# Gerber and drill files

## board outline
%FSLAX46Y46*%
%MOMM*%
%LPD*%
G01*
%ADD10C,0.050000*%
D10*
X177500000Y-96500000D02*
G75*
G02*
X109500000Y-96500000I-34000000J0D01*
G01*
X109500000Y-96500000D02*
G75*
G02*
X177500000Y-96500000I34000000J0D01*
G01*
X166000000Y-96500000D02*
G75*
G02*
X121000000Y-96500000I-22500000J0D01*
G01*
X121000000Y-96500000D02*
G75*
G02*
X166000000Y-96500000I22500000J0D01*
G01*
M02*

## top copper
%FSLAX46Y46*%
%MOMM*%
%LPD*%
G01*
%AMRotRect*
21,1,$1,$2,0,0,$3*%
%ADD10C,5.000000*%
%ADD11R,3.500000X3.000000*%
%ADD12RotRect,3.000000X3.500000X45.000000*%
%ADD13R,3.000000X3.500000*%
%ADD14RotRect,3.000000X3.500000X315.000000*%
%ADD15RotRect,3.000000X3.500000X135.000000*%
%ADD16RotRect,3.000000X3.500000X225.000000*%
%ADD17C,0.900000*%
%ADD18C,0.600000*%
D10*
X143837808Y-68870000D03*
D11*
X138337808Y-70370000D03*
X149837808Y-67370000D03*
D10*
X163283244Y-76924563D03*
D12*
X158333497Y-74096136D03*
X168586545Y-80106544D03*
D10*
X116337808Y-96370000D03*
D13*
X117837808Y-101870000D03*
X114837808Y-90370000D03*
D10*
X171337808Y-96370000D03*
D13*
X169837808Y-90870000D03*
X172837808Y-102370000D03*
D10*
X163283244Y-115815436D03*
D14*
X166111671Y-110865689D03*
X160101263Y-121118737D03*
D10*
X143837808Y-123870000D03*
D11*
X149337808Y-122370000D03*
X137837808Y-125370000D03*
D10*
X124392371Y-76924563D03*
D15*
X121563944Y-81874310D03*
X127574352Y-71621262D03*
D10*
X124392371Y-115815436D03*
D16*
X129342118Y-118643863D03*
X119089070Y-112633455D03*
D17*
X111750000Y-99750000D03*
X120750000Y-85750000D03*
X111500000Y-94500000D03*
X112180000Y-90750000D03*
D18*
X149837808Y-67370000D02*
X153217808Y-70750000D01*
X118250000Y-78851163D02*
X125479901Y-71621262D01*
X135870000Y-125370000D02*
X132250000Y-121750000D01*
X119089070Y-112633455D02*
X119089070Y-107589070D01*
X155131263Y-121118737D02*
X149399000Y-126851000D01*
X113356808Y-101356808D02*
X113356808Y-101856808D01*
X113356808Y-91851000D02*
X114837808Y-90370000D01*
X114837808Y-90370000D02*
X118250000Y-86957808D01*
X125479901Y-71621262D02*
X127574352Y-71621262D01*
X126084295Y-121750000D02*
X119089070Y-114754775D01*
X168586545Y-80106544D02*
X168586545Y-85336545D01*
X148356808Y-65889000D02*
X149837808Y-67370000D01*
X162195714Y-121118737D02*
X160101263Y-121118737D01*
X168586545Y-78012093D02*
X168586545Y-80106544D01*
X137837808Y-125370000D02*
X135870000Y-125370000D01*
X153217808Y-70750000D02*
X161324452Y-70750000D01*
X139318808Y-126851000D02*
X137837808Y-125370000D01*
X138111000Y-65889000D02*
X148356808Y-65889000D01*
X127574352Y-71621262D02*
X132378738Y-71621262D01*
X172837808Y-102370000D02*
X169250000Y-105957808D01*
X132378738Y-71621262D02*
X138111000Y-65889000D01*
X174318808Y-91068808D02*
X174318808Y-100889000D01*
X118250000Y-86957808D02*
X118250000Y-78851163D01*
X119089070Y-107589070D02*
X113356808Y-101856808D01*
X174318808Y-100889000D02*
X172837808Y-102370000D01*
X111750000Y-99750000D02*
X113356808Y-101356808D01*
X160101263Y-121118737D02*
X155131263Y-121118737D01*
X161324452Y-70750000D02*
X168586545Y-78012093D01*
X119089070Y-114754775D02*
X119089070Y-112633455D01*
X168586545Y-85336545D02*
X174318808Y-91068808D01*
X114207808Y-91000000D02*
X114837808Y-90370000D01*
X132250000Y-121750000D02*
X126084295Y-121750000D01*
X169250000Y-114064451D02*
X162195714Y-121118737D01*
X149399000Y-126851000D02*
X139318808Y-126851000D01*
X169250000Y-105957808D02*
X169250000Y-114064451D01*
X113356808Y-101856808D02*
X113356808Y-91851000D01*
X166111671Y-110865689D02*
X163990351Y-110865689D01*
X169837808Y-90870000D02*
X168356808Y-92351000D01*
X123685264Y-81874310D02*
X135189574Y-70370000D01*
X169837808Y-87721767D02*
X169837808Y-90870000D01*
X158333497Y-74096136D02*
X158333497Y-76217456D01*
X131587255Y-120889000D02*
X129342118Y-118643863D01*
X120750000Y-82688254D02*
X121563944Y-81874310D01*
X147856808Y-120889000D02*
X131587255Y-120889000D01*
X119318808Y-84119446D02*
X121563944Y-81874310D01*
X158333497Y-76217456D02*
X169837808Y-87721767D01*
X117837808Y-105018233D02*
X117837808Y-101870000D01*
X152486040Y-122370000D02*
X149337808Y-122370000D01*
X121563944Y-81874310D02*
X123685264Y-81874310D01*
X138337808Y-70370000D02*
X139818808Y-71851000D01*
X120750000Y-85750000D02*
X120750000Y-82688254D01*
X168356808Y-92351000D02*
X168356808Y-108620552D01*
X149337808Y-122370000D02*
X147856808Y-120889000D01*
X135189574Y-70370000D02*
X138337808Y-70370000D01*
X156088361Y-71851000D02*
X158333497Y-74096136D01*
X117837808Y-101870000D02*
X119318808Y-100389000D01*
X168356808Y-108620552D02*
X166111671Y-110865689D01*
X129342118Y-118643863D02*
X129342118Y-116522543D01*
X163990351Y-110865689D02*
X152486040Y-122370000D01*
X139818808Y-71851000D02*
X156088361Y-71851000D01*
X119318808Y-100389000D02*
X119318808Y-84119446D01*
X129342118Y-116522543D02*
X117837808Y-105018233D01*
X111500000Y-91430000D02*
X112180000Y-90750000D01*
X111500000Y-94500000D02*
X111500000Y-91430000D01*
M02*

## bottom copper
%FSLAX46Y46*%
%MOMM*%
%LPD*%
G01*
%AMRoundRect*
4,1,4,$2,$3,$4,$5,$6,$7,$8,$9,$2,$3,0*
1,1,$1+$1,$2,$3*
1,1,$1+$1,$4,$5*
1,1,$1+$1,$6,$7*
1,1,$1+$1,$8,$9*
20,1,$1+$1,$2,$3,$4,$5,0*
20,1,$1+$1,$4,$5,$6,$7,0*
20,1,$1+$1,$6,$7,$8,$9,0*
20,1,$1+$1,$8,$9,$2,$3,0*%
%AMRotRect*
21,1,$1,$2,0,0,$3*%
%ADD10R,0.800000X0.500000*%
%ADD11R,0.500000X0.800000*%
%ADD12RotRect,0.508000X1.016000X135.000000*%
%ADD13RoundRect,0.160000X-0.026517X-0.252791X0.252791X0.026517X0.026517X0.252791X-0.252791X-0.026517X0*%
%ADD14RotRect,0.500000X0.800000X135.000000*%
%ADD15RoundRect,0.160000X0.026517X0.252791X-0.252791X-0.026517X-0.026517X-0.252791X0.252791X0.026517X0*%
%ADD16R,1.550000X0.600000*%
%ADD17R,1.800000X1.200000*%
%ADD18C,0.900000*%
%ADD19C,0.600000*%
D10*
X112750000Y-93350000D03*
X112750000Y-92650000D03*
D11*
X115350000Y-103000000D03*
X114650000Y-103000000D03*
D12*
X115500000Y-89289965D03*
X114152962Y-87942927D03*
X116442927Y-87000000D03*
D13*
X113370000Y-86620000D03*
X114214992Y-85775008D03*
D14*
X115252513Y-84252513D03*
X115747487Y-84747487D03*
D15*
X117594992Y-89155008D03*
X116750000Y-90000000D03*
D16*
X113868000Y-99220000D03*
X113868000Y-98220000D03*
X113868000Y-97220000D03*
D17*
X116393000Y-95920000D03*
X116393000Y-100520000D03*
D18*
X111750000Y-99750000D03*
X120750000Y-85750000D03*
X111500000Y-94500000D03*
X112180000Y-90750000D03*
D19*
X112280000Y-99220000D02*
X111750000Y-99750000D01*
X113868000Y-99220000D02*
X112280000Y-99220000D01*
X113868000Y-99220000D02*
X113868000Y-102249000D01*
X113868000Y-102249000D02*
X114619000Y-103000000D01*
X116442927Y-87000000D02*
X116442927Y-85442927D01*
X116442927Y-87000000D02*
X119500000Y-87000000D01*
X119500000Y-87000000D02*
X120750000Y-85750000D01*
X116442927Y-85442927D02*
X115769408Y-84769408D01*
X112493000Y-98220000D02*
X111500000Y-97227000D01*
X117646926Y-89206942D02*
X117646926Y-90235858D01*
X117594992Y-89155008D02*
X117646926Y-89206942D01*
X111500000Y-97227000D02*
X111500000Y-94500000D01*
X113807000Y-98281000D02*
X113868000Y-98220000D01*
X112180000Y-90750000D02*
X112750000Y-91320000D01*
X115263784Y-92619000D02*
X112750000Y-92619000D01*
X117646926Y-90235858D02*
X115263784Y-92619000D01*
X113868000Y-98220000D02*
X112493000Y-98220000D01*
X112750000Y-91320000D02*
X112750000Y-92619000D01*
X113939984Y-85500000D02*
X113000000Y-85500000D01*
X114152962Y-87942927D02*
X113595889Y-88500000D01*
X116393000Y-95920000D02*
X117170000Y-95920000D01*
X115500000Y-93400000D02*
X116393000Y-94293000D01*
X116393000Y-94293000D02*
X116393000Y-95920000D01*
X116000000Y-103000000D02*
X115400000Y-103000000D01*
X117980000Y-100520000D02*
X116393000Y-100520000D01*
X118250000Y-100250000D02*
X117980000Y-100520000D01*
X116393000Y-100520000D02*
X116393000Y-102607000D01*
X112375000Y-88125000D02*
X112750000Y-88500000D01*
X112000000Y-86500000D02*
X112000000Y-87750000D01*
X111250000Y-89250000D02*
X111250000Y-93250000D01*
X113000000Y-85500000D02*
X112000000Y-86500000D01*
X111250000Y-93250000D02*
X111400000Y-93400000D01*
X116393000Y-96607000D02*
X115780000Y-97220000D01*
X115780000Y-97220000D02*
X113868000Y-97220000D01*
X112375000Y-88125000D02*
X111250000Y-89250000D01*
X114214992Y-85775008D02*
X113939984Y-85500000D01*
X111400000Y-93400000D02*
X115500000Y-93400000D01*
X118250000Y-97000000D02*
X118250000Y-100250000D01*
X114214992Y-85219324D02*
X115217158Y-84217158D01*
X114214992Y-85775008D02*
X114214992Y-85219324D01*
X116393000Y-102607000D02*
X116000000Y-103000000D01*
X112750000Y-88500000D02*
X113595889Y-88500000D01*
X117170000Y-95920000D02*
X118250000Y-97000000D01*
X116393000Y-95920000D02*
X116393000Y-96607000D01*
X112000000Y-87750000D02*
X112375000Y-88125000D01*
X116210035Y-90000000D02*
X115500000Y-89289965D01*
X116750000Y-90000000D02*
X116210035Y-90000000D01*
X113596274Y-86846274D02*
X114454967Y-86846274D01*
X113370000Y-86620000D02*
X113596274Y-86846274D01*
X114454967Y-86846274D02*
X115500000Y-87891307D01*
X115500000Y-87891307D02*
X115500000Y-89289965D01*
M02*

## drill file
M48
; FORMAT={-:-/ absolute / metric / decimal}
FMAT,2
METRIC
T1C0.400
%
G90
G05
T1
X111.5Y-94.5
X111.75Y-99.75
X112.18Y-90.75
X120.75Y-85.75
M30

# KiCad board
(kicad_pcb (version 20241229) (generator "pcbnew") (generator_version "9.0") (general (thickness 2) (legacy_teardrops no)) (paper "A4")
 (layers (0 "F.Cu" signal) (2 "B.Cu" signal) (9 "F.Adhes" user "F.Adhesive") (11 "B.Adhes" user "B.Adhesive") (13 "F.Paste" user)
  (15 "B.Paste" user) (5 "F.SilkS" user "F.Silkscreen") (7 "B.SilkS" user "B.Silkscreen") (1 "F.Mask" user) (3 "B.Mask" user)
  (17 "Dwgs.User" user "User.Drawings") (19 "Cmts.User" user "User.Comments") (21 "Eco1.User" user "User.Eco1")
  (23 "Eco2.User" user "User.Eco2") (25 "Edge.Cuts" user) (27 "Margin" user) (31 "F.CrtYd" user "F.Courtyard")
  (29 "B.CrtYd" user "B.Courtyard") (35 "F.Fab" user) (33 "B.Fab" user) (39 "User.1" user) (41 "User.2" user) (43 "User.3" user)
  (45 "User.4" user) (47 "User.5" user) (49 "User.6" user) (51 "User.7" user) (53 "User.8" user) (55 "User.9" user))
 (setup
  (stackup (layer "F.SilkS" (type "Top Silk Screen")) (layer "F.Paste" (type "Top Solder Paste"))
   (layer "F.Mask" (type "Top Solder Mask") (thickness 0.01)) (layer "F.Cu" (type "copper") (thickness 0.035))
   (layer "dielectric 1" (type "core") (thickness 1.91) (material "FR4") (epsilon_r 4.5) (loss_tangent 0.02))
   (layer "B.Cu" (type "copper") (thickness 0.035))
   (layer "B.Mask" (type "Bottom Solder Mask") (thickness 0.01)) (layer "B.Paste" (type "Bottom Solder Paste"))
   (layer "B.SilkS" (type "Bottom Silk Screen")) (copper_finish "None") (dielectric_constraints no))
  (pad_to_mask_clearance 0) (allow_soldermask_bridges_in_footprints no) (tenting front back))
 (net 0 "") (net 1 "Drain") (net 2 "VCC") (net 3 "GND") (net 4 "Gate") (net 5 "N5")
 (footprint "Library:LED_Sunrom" (layer "F.Cu") (at 143.837808 68.87)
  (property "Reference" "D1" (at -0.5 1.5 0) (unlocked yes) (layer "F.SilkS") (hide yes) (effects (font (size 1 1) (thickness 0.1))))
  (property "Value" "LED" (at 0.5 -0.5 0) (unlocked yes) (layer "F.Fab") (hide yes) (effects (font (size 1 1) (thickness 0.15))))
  (pad "" smd circle (at 0 0 90) (size 5 5) (layers "F.Cu" "F.Mask" "F.Paste") (solder_mask_margin 0.102))
  (pad "1" smd rect (at -5.5 1.5 90) (size 3 3.5) (layers "F.Cu" "F.Mask" "F.Paste") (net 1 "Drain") (solder_mask_margin 0.102))
  (pad "2" smd rect (at 6 -1.5 90) (size 3 3.5) (layers "F.Cu" "F.Mask" "F.Paste") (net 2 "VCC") (solder_mask_margin 0.102)))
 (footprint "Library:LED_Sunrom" (layer "F.Cu") (at 163.283244 76.924563 -45)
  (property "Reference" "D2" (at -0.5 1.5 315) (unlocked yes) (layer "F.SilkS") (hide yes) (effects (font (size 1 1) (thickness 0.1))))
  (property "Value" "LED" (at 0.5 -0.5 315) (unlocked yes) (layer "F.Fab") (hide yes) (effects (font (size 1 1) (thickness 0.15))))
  (pad "" smd circle (at 0 0 45) (size 5 5) (layers "F.Cu" "F.Mask" "F.Paste") (solder_mask_margin 0.102))
  (pad "1" smd rect (at -5.5 1.5 45) (size 3 3.5) (layers "F.Cu" "F.Mask" "F.Paste") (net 1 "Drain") (solder_mask_margin 0.102))
  (pad "2" smd rect (at 6 -1.5 45) (size 3 3.5) (layers "F.Cu" "F.Mask" "F.Paste") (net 2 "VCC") (solder_mask_margin 0.102)))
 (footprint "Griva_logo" (layer "F.Cu") (at 116.847808 106.51)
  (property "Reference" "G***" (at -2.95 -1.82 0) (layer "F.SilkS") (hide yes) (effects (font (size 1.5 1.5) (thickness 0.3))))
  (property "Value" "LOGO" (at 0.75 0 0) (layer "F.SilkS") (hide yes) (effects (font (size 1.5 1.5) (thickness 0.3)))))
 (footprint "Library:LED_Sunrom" (layer "F.Cu") (at 116.337808 96.37 90)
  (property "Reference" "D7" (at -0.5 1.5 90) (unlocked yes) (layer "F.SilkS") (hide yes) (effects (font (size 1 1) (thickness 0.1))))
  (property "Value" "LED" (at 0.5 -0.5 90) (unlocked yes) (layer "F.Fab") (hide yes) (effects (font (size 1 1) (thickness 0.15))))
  (pad "" smd circle (at 0 0 180) (size 5 5) (layers "F.Cu" "F.Mask" "F.Paste") (solder_mask_margin 0.102))
  (pad "1" smd rect (at -5.5 1.5 180) (size 3 3.5) (layers "F.Cu" "F.Mask" "F.Paste") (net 1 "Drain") (solder_mask_margin 0.102))
  (pad "2" smd rect (at 6 -1.5 180) (size 3 3.5) (layers "F.Cu" "F.Mask" "F.Paste") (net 2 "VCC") (solder_mask_margin 0.102)))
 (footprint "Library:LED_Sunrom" (layer "F.Cu") (at 171.337808 96.37 -90)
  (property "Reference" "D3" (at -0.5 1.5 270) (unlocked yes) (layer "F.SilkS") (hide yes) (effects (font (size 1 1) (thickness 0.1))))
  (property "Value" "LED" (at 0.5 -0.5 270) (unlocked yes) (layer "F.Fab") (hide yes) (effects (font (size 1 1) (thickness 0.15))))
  (pad "" smd circle (at 0 0) (size 5 5) (layers "F.Cu" "F.Mask" "F.Paste") (solder_mask_margin 0.102))
  (pad "1" smd rect (at -5.5 1.5) (size 3 3.5) (layers "F.Cu" "F.Mask" "F.Paste") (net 1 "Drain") (solder_mask_margin 0.102))
  (pad "2" smd rect (at 6 -1.5) (size 3 3.5) (layers "F.Cu" "F.Mask" "F.Paste") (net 2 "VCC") (solder_mask_margin 0.102)))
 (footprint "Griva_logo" (layer "F.Cu") (at 23.59 18.28)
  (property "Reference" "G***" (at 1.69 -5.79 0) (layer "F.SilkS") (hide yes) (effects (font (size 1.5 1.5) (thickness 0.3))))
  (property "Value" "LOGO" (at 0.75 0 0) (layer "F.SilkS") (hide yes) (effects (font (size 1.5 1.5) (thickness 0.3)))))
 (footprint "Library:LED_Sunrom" (layer "F.Cu") (at 163.283244 115.815436 -135)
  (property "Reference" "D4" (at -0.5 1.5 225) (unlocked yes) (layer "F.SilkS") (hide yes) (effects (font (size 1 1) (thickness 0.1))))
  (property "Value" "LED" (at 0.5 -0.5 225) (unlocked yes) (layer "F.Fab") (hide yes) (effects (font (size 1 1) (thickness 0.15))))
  (pad "" smd circle (at 0 0 315) (size 5 5) (layers "F.Cu" "F.Mask" "F.Paste") (solder_mask_margin 0.102))
  (pad "1" smd rect (at -5.5 1.5 315) (size 3 3.5) (layers "F.Cu" "F.Mask" "F.Paste") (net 1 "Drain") (solder_mask_margin 0.102))
  (pad "2" smd rect (at 6 -1.5 315) (size 3 3.5) (layers "F.Cu" "F.Mask" "F.Paste") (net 2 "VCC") (solder_mask_margin 0.102)))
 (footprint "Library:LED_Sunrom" (layer "F.Cu") (at 143.837808 123.87 180)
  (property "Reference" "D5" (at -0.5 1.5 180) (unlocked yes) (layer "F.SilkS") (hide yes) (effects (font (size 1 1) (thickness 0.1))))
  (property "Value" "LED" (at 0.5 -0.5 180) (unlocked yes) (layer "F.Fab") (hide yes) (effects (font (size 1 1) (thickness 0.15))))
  (pad "" smd circle (at 0 0 270) (size 5 5) (layers "F.Cu" "F.Mask" "F.Paste") (solder_mask_margin 0.102))
  (pad "1" smd rect (at -5.5 1.5 270) (size 3 3.5) (layers "F.Cu" "F.Mask" "F.Paste") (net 1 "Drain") (solder_mask_margin 0.102))
  (pad "2" smd rect (at 6 -1.5 270) (size 3 3.5) (layers "F.Cu" "F.Mask" "F.Paste") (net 2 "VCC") (solder_mask_margin 0.102)))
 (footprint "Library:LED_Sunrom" (layer "F.Cu") (at 124.392371 76.924563 45)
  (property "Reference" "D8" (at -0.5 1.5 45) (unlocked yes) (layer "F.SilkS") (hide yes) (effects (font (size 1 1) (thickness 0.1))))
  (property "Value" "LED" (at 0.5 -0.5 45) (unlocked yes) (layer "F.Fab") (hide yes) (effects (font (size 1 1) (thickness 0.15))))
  (pad "" smd circle (at 0 0 135) (size 5 5) (layers "F.Cu" "F.Mask" "F.Paste") (solder_mask_margin 0.102))
  (pad "1" smd rect (at -5.5 1.5 135) (size 3 3.5) (layers "F.Cu" "F.Mask" "F.Paste") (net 1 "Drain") (solder_mask_margin 0.102))
  (pad "2" smd rect (at 6 -1.5 135) (size 3 3.5) (layers "F.Cu" "F.Mask" "F.Paste") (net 2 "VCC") (solder_mask_margin 0.102)))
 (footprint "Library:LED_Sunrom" (layer "F.Cu") (at 124.392371 115.815436 135)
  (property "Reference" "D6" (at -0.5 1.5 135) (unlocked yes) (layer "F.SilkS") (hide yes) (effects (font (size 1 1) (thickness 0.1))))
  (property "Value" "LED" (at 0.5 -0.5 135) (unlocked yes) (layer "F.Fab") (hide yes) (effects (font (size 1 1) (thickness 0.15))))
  (pad "" smd circle (at 0 0 225) (size 5 5) (layers "F.Cu" "F.Mask" "F.Paste") (solder_mask_margin 0.102))
  (pad "1" smd rect (at -5.5 1.5 225) (size 3 3.5) (layers "F.Cu" "F.Mask" "F.Paste") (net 1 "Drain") (solder_mask_margin 0.102))
  (pad "2" smd rect (at 6 -1.5 225) (size 3 3.5) (layers "F.Cu" "F.Mask" "F.Paste") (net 2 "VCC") (solder_mask_margin 0.102)))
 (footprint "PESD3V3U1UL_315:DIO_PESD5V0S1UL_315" (layer "B.Cu") (at 112.75 93 -90)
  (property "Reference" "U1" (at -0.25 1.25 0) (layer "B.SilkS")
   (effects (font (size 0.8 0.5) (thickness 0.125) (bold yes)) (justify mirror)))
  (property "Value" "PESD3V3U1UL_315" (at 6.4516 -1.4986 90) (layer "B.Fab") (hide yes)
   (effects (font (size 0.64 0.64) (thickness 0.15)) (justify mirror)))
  (pad "A" smd rect (at 0.35 0 270) (size 0.5 0.8) (layers "B.Cu") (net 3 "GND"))
  (pad "K" smd rect (at -0.35 0 270) (size 0.5 0.8) (layers "B.Cu") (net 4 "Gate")))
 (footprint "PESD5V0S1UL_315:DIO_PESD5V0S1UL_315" (layer "B.Cu") (at 115 103)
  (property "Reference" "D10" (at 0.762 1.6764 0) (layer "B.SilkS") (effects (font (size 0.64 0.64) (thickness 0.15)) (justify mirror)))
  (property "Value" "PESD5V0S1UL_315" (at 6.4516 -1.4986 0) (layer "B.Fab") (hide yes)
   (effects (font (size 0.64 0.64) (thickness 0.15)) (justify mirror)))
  (pad "A" smd rect (at 0.35 0) (size 0.5 0.8) (layers "B.Cu") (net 3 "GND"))
  (pad "K" smd rect (at -0.35 0) (size 0.5 0.8) (layers "B.Cu") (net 2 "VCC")))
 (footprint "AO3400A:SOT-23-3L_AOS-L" (layer "B.Cu") (at 115.634704 87.808223 135)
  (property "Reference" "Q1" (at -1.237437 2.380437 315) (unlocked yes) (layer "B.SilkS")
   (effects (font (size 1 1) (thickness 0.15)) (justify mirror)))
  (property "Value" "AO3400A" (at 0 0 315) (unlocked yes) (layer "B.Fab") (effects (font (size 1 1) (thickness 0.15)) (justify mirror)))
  (pad "1" smd rect (at -0.9525 -1.143 135) (size 0.508 1.016) (layers "B.Cu" "B.Mask" "B.Paste") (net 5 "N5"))
  (pad "2" smd rect (at 0.9525 -1.143 135) (size 0.508 1.016) (layers "B.Cu" "B.Mask" "B.Paste") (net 3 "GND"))
  (pad "3" smd rect (at 0 1.143 135) (size 0.508 1.016) (layers "B.Cu" "B.Mask" "B.Paste") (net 1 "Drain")))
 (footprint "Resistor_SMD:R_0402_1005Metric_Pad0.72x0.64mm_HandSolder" (layer "B.Cu") (at 113.792496 86.197504 45)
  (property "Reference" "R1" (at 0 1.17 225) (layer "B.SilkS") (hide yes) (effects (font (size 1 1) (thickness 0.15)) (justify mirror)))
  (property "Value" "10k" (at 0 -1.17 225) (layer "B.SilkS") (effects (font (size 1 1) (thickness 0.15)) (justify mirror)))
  (pad "1" smd roundrect (at -0.5975 0 45) (size 0.715 0.64) (layers "B.Cu" "B.Mask" "B.Paste") (roundrect_rratio 0.25) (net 5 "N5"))
  (pad "2" smd roundrect (at 0.5975 0 45) (size 0.715 0.64) (layers "B.Cu" "B.Mask" "B.Paste") (roundrect_rratio 0.25) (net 3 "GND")))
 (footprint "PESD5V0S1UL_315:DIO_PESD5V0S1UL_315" (layer "B.Cu") (at 115.5 84.5 135)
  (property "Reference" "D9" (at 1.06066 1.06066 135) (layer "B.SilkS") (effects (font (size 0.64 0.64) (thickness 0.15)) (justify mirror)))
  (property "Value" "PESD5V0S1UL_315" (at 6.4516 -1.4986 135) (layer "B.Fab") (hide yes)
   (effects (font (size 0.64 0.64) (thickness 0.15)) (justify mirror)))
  (pad "A" smd rect (at 0.349999 0 135) (size 0.5 0.8) (layers "B.Cu") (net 3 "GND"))
  (pad "K" smd rect (at -0.349999 0 135) (size 0.5 0.8) (layers "B.Cu") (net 1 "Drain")))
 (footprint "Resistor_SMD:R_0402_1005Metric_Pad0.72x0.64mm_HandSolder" (layer "B.Cu") (at 117.172496 89.577504 -135)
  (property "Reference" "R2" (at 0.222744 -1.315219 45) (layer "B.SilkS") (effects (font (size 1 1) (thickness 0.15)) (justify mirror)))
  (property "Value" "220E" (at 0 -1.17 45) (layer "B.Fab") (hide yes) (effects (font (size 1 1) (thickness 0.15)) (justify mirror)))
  (pad "1" smd roundrect (at -0.5975 0 225) (size 0.715 0.64) (layers "B.Cu" "B.Mask" "B.Paste") (roundrect_rratio 0.25) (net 4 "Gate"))
  (pad "2" smd roundrect (at 0.5975 0 225) (size 0.715 0.64) (layers "B.Cu" "B.Mask" "B.Paste") (roundrect_rratio 0.25) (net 5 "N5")))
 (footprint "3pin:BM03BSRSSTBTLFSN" (layer "B.Cu") (at 115.48 98.22 -90)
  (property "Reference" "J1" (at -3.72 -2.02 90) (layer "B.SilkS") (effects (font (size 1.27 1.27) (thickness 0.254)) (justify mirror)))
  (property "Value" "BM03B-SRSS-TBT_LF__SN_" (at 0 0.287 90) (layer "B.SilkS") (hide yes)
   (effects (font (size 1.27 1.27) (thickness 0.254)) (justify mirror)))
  (pad "1" smd rect (at 1 1.612 270) (size 0.6 1.55) (layers "B.Cu" "B.Mask" "B.Paste") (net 2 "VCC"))
  (pad "2" smd rect (at 0 1.612 270) (size 0.6 1.55) (layers "B.Cu" "B.Mask" "B.Paste") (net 4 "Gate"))
  (pad "3" smd rect (at -1 1.612 270) (size 0.6 1.55) (layers "B.Cu" "B.Mask" "B.Paste") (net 3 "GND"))
  (pad "4" smd rect (at -2.3 -0.913 270) (size 1.2 1.8) (layers "B.Cu" "B.Mask" "B.Paste") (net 3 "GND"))
  (pad "5" smd rect (at 2.3 -0.913 270) (size 1.2 1.8) (layers "B.Cu" "B.Mask" "B.Paste") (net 3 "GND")))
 (gr_circle (center 143.5 96.5) (end 177.5 96.5) (stroke (width 0.05) (type solid)) (fill no) (layer "Edge.Cuts"))
 (gr_circle (center 143.5 96.5) (end 166 96.5) (stroke (width 0.05) (type default)) (fill no) (layer "Edge.Cuts"))
 (segment (start 149.837808 67.37) (end 153.217808 70.75) (width 0.6) (layer "F.Cu") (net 2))
 (segment (start 118.25 78.851163) (end 125.479901 71.621262) (width 0.6) (layer "F.Cu") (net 2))
 (segment (start 135.87 125.37) (end 132.25 121.75) (width 0.6) (layer "F.Cu") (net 2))
 (segment (start 119.08907 112.633455) (end 119.08907 107.58907) (width 0.6) (layer "F.Cu") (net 2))
 (segment (start 155.131263 121.118737) (end 149.399 126.851) (width 0.6) (layer "F.Cu") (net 2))
 (segment (start 113.356808 101.356808) (end 113.356808 101.856808) (width 0.6) (layer "F.Cu") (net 2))
 (segment (start 113.356808 91.851) (end 114.837808 90.37) (width 0.6) (layer "F.Cu") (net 2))
 (segment (start 114.837808 90.37) (end 118.25 86.957808) (width 0.6) (layer "F.Cu") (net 2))
 (segment (start 125.479901 71.621262) (end 127.574352 71.621262) (width 0.6) (layer "F.Cu") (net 2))
 (segment (start 126.084295 121.75) (end 119.08907 114.754775) (width 0.6) (layer "F.Cu") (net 2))
 (segment (start 168.586545 80.106544) (end 168.586545 85.336545) (width 0.6) (layer "F.Cu") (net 2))
 (segment (start 148.356808 65.889) (end 149.837808 67.37) (width 0.6) (layer "F.Cu") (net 2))
 (segment (start 162.195714 121.118737) (end 160.101263 121.118737) (width 0.6) (layer "F.Cu") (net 2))
 (segment (start 168.586545 78.012093) (end 168.586545 80.106544) (width 0.6) (layer "F.Cu") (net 2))
 (segment (start 137.837808 125.37) (end 135.87 125.37) (width 0.6) (layer "F.Cu") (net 2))
 (segment (start 153.217808 70.75) (end 161.324452 70.75) (width 0.6) (layer "F.Cu") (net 2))
 (segment (start 139.318808 126.851) (end 137.837808 125.37) (width 0.6) (layer "F.Cu") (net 2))
 (segment (start 138.111 65.889) (end 148.356808 65.889) (width 0.6) (layer "F.Cu") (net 2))
 (segment (start 127.574352 71.621262) (end 132.378738 71.621262) (width 0.6) (layer "F.Cu") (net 2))
 (segment (start 172.837808 102.37) (end 169.25 105.957808) (width 0.6) (layer "F.Cu") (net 2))
 (segment (start 132.378738 71.621262) (end 138.111 65.889) (width 0.6) (layer "F.Cu") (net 2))
 (segment (start 174.318808 91.068808) (end 174.318808 100.889) (width 0.6) (layer "F.Cu") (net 2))
 (segment (start 118.25 86.957808) (end 118.25 78.851163) (width 0.6) (layer "F.Cu") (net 2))
 (segment (start 119.08907 107.58907) (end 113.356808 101.856808) (width 0.6) (layer "F.Cu") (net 2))
 (segment (start 174.318808 100.889) (end 172.837808 102.37) (width 0.6) (layer "F.Cu") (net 2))
 (segment (start 111.75 99.75) (end 113.356808 101.356808) (width 0.6) (layer "F.Cu") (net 2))
 (segment (start 160.101263 121.118737) (end 155.131263 121.118737) (width 0.6) (layer "F.Cu") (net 2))
 (segment (start 161.324452 70.75) (end 168.586545 78.012093) (width 0.6) (layer "F.Cu") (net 2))
 (segment (start 119.08907 114.754775) (end 119.08907 112.633455) (width 0.6) (layer "F.Cu") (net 2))
 (segment (start 168.586545 85.336545) (end 174.318808 91.068808) (width 0.6) (layer "F.Cu") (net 2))
 (segment (start 114.207808 91) (end 114.837808 90.37) (width 0.6) (layer "F.Cu") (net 2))
 (segment (start 132.25 121.75) (end 126.084295 121.75) (width 0.6) (layer "F.Cu") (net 2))
 (segment (start 169.25 114.064451) (end 162.195714 121.118737) (width 0.6) (layer "F.Cu") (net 2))
 (segment (start 149.399 126.851) (end 139.318808 126.851) (width 0.6) (layer "F.Cu") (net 2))
 (segment (start 169.25 105.957808) (end 169.25 114.064451) (width 0.6) (layer "F.Cu") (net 2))
 (segment (start 113.356808 101.856808) (end 113.356808 91.851) (width 0.6) (layer "F.Cu") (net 2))
 (via (at 111.75 99.75) (size 0.9) (drill 0.4) (layers "F.Cu" "B.Cu") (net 2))
 (segment (start 112.28 99.22) (end 111.75 99.75) (width 0.6) (layer "B.Cu") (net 2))
 (segment (start 113.868 99.22) (end 112.28 99.22) (width 0.6) (layer "B.Cu") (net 2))
 (segment (start 113.868 99.22) (end 113.868 102.249) (width 0.6) (layer "B.Cu") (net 2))
 (segment (start 113.868 102.249) (end 114.619 103) (width 0.6) (layer "B.Cu") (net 2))
 (segment (start 166.111671 110.865689) (end 163.990351 110.865689) (width 0.6) (layer "F.Cu") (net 1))
 (segment (start 169.837808 90.87) (end 168.356808 92.351) (width 0.6) (layer "F.Cu") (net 1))
 (segment (start 123.685264 81.87431) (end 135.189574 70.37) (width 0.6) (layer "F.Cu") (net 1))
 (segment (start 169.837808 87.721767) (end 169.837808 90.87) (width 0.6) (layer "F.Cu") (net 1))
 (segment (start 158.333497 74.096136) (end 158.333497 76.217456) (width 0.6) (layer "F.Cu") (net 1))
 (segment (start 131.587255 120.889) (end 129.342118 118.643863) (width 0.6) (layer "F.Cu") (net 1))
 (segment (start 120.75 82.688254) (end 121.563944 81.87431) (width 0.6) (layer "F.Cu") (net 1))
 (segment (start 147.856808 120.889) (end 131.587255 120.889) (width 0.6) (layer "F.Cu") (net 1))
 (segment (start 119.318808 84.119446) (end 121.563944 81.87431) (width 0.6) (layer "F.Cu") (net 1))
 (segment (start 158.333497 76.217456) (end 169.837808 87.721767) (width 0.6) (layer "F.Cu") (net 1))
 (segment (start 117.837808 105.018233) (end 117.837808 101.87) (width 0.6) (layer "F.Cu") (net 1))
 (segment (start 152.48604 122.37) (end 149.337808 122.37) (width 0.6) (layer "F.Cu") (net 1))
 (segment (start 121.563944 81.87431) (end 123.685264 81.87431) (width 0.6) (layer "F.Cu") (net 1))
 (segment (start 138.337808 70.37) (end 139.818808 71.851) (width 0.6) (layer "F.Cu") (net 1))
 (segment (start 120.75 85.75) (end 120.75 82.688254) (width 0.6) (layer "F.Cu") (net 1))
 (segment (start 168.356808 92.351) (end 168.356808 108.620552) (width 0.6) (layer "F.Cu") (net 1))
 (segment (start 149.337808 122.37) (end 147.856808 120.889) (width 0.6) (layer "F.Cu") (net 1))
 (segment (start 135.189574 70.37) (end 138.337808 70.37) (width 0.6) (layer "F.Cu") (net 1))
 (segment (start 156.088361 71.851) (end 158.333497 74.096136) (width 0.6) (layer "F.Cu") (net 1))
 (segment (start 117.837808 101.87) (end 119.318808 100.389) (width 0.6) (layer "F.Cu") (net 1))
 (segment (start 168.356808 108.620552) (end 166.111671 110.865689) (width 0.6) (layer "F.Cu") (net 1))
 (segment (start 129.342118 118.643863) (end 129.342118 116.522543) (width 0.6) (layer "F.Cu") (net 1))
 (segment (start 163.990351 110.865689) (end 152.48604 122.37) (width 0.6) (layer "F.Cu") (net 1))
 (segment (start 139.818808 71.851) (end 156.088361 71.851) (width 0.6) (layer "F.Cu") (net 1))
 (segment (start 119.318808 100.389) (end 119.318808 84.119446) (width 0.6) (layer "F.Cu") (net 1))
 (segment (start 129.342118 116.522543) (end 117.837808 105.018233) (width 0.6) (layer "F.Cu") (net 1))
 (via (at 120.75 85.75) (size 0.9) (drill 0.4) (layers "F.Cu" "B.Cu") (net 1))
 (segment (start 116.442927 87) (end 116.442927 85.442927) (width 0.6) (layer "B.Cu") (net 1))
 (segment (start 116.442927 87) (end 119.5 87) (width 0.6) (layer "B.Cu") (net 1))
 (segment (start 119.5 87) (end 120.75 85.75) (width 0.6) (layer "B.Cu") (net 1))
 (segment (start 116.442927 85.442927) (end 115.769408 84.769408) (width 0.6) (layer "B.Cu") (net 1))
 (segment (start 111.5 91.43) (end 112.18 90.75) (width 0.6) (layer "F.Cu") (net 4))
 (segment (start 111.5 94.5) (end 111.5 91.43) (width 0.6) (layer "F.Cu") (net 4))
 (via (at 111.5 94.5) (size 0.9) (drill 0.4) (layers "F.Cu" "B.Cu") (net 4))
 (via (at 112.18 90.75) (size 0.9) (drill 0.4) (layers "F.Cu" "B.Cu") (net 4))
 (segment (start 112.493 98.22) (end 111.5 97.227) (width 0.6) (layer "B.Cu") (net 4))
 (segment (start 117.646926 89.206942) (end 117.646926 90.235858) (width 0.6) (layer "B.Cu") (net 4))
 (segment (start 117.594992 89.155008) (end 117.646926 89.206942) (width 0.6) (layer "B.Cu") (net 4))
 (segment (start 111.5 97.227) (end 111.5 94.5) (width 0.6) (layer "B.Cu") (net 4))
 (segment (start 113.807 98.281) (end 113.868 98.22) (width 0.6) (layer "B.Cu") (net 4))
 (segment (start 112.18 90.75) (end 112.75 91.32) (width 0.6) (layer "B.Cu") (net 4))
 (segment (start 115.263784 92.619) (end 112.75 92.619) (width 0.6) (layer "B.Cu") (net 4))
 (segment (start 117.646926 90.235858) (end 115.263784 92.619) (width 0.6) (layer "B.Cu") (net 4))
 (segment (start 113.868 98.22) (end 112.493 98.22) (width 0.6) (layer "B.Cu") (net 4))
 (segment (start 112.75 91.32) (end 112.75 92.619) (width 0.6) (layer "B.Cu") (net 4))
 (segment (start 113.939984 85.5) (end 113 85.5) (width 0.6) (layer "B.Cu") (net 3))
 (segment (start 114.152962 87.942927) (end 113.595889 88.5) (width 0.6) (layer "B.Cu") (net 3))
 (segment (start 116.393 95.92) (end 117.17 95.92) (width 0.6) (layer "B.Cu") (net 3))
 (segment (start 115.5 93.4) (end 116.393 94.293) (width 0.6) (layer "B.Cu") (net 3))
 (segment (start 116.393 94.293) (end 116.393 95.92) (width 0.6) (layer "B.Cu") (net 3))
 (segment (start 116 103) (end 115.4 103) (width 0.6) (layer "B.Cu") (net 3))
 (segment (start 117.98 100.52) (end 116.393 100.52) (width 0.6) (layer "B.Cu") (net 3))
 (segment (start 118.25 100.25) (end 117.98 100.52) (width 0.6) (layer "B.Cu") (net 3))
 (segment (start 116.393 100.52) (end 116.393 102.607) (width 0.6) (layer "B.Cu") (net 3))
 (segment (start 112.375 88.125) (end 112.75 88.5) (width 0.6) (layer "B.Cu") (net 3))
 (segment (start 112 86.5) (end 112 87.75) (width 0.6) (layer "B.Cu") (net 3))
 (segment (start 111.25 89.25) (end 111.25 93.25) (width 0.6) (layer "B.Cu") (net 3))
 (segment (start 113 85.5) (end 112 86.5) (width 0.6) (layer "B.Cu") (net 3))
 (segment (start 111.25 93.25) (end 111.4 93.4) (width 0.6) (layer "B.Cu") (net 3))
 (segment (start 116.393 96.607) (end 115.78 97.22) (width 0.6) (layer "B.Cu") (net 3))
 (segment (start 115.78 97.22) (end 113.868 97.22) (width 0.6) (layer "B.Cu") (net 3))
 (segment (start 112.375 88.125) (end 111.25 89.25) (width 0.6) (layer "B.Cu") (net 3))
 (segment (start 114.214992 85.775008) (end 113.939984 85.5) (width 0.6) (layer "B.Cu") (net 3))
 (segment (start 111.4 93.4) (end 115.5 93.4) (width 0.6) (layer "B.Cu") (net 3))
 (segment (start 118.25 97) (end 118.25 100.25) (width 0.6) (layer "B.Cu") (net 3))
 (segment (start 114.214992 85.219324) (end 115.217158 84.217158) (width 0.6) (layer "B.Cu") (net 3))
 (segment (start 114.214992 85.775008) (end 114.214992 85.219324) (width 0.6) (layer "B.Cu") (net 3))
 (segment (start 116.393 102.607) (end 116 103) (width 0.6) (layer "B.Cu") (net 3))
 (segment (start 112.75 88.5) (end 113.595889 88.5) (width 0.6) (layer "B.Cu") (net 3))
 (segment (start 117.17 95.92) (end 118.25 97) (width 0.6) (layer "B.Cu") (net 3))
 (segment (start 116.393 95.92) (end 116.393 96.607) (width 0.6) (layer "B.Cu") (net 3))
 (segment (start 112 87.75) (end 112.375 88.125) (width 0.6) (layer "B.Cu") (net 3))
 (segment (start 116.210035 90) (end 115.5 89.289965) (width 0.6) (layer "B.Cu") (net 5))
 (segment (start 116.75 90) (end 116.210035 90) (width 0.6) (layer "B.Cu") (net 5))
 (segment (start 113.596274 86.846274) (end 114.454967 86.846274) (width 0.6) (layer "B.Cu") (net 5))
 (segment (start 113.37 86.62) (end 113.596274 86.846274) (width 0.6) (layer "B.Cu") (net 5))
 (segment (start 114.454967 86.846274) (end 115.5 87.891307) (width 0.6) (layer "B.Cu") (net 5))
 (segment (start 115.5 87.891307) (end 115.5 89.289965) (width 0.6) (layer "B.Cu") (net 5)))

